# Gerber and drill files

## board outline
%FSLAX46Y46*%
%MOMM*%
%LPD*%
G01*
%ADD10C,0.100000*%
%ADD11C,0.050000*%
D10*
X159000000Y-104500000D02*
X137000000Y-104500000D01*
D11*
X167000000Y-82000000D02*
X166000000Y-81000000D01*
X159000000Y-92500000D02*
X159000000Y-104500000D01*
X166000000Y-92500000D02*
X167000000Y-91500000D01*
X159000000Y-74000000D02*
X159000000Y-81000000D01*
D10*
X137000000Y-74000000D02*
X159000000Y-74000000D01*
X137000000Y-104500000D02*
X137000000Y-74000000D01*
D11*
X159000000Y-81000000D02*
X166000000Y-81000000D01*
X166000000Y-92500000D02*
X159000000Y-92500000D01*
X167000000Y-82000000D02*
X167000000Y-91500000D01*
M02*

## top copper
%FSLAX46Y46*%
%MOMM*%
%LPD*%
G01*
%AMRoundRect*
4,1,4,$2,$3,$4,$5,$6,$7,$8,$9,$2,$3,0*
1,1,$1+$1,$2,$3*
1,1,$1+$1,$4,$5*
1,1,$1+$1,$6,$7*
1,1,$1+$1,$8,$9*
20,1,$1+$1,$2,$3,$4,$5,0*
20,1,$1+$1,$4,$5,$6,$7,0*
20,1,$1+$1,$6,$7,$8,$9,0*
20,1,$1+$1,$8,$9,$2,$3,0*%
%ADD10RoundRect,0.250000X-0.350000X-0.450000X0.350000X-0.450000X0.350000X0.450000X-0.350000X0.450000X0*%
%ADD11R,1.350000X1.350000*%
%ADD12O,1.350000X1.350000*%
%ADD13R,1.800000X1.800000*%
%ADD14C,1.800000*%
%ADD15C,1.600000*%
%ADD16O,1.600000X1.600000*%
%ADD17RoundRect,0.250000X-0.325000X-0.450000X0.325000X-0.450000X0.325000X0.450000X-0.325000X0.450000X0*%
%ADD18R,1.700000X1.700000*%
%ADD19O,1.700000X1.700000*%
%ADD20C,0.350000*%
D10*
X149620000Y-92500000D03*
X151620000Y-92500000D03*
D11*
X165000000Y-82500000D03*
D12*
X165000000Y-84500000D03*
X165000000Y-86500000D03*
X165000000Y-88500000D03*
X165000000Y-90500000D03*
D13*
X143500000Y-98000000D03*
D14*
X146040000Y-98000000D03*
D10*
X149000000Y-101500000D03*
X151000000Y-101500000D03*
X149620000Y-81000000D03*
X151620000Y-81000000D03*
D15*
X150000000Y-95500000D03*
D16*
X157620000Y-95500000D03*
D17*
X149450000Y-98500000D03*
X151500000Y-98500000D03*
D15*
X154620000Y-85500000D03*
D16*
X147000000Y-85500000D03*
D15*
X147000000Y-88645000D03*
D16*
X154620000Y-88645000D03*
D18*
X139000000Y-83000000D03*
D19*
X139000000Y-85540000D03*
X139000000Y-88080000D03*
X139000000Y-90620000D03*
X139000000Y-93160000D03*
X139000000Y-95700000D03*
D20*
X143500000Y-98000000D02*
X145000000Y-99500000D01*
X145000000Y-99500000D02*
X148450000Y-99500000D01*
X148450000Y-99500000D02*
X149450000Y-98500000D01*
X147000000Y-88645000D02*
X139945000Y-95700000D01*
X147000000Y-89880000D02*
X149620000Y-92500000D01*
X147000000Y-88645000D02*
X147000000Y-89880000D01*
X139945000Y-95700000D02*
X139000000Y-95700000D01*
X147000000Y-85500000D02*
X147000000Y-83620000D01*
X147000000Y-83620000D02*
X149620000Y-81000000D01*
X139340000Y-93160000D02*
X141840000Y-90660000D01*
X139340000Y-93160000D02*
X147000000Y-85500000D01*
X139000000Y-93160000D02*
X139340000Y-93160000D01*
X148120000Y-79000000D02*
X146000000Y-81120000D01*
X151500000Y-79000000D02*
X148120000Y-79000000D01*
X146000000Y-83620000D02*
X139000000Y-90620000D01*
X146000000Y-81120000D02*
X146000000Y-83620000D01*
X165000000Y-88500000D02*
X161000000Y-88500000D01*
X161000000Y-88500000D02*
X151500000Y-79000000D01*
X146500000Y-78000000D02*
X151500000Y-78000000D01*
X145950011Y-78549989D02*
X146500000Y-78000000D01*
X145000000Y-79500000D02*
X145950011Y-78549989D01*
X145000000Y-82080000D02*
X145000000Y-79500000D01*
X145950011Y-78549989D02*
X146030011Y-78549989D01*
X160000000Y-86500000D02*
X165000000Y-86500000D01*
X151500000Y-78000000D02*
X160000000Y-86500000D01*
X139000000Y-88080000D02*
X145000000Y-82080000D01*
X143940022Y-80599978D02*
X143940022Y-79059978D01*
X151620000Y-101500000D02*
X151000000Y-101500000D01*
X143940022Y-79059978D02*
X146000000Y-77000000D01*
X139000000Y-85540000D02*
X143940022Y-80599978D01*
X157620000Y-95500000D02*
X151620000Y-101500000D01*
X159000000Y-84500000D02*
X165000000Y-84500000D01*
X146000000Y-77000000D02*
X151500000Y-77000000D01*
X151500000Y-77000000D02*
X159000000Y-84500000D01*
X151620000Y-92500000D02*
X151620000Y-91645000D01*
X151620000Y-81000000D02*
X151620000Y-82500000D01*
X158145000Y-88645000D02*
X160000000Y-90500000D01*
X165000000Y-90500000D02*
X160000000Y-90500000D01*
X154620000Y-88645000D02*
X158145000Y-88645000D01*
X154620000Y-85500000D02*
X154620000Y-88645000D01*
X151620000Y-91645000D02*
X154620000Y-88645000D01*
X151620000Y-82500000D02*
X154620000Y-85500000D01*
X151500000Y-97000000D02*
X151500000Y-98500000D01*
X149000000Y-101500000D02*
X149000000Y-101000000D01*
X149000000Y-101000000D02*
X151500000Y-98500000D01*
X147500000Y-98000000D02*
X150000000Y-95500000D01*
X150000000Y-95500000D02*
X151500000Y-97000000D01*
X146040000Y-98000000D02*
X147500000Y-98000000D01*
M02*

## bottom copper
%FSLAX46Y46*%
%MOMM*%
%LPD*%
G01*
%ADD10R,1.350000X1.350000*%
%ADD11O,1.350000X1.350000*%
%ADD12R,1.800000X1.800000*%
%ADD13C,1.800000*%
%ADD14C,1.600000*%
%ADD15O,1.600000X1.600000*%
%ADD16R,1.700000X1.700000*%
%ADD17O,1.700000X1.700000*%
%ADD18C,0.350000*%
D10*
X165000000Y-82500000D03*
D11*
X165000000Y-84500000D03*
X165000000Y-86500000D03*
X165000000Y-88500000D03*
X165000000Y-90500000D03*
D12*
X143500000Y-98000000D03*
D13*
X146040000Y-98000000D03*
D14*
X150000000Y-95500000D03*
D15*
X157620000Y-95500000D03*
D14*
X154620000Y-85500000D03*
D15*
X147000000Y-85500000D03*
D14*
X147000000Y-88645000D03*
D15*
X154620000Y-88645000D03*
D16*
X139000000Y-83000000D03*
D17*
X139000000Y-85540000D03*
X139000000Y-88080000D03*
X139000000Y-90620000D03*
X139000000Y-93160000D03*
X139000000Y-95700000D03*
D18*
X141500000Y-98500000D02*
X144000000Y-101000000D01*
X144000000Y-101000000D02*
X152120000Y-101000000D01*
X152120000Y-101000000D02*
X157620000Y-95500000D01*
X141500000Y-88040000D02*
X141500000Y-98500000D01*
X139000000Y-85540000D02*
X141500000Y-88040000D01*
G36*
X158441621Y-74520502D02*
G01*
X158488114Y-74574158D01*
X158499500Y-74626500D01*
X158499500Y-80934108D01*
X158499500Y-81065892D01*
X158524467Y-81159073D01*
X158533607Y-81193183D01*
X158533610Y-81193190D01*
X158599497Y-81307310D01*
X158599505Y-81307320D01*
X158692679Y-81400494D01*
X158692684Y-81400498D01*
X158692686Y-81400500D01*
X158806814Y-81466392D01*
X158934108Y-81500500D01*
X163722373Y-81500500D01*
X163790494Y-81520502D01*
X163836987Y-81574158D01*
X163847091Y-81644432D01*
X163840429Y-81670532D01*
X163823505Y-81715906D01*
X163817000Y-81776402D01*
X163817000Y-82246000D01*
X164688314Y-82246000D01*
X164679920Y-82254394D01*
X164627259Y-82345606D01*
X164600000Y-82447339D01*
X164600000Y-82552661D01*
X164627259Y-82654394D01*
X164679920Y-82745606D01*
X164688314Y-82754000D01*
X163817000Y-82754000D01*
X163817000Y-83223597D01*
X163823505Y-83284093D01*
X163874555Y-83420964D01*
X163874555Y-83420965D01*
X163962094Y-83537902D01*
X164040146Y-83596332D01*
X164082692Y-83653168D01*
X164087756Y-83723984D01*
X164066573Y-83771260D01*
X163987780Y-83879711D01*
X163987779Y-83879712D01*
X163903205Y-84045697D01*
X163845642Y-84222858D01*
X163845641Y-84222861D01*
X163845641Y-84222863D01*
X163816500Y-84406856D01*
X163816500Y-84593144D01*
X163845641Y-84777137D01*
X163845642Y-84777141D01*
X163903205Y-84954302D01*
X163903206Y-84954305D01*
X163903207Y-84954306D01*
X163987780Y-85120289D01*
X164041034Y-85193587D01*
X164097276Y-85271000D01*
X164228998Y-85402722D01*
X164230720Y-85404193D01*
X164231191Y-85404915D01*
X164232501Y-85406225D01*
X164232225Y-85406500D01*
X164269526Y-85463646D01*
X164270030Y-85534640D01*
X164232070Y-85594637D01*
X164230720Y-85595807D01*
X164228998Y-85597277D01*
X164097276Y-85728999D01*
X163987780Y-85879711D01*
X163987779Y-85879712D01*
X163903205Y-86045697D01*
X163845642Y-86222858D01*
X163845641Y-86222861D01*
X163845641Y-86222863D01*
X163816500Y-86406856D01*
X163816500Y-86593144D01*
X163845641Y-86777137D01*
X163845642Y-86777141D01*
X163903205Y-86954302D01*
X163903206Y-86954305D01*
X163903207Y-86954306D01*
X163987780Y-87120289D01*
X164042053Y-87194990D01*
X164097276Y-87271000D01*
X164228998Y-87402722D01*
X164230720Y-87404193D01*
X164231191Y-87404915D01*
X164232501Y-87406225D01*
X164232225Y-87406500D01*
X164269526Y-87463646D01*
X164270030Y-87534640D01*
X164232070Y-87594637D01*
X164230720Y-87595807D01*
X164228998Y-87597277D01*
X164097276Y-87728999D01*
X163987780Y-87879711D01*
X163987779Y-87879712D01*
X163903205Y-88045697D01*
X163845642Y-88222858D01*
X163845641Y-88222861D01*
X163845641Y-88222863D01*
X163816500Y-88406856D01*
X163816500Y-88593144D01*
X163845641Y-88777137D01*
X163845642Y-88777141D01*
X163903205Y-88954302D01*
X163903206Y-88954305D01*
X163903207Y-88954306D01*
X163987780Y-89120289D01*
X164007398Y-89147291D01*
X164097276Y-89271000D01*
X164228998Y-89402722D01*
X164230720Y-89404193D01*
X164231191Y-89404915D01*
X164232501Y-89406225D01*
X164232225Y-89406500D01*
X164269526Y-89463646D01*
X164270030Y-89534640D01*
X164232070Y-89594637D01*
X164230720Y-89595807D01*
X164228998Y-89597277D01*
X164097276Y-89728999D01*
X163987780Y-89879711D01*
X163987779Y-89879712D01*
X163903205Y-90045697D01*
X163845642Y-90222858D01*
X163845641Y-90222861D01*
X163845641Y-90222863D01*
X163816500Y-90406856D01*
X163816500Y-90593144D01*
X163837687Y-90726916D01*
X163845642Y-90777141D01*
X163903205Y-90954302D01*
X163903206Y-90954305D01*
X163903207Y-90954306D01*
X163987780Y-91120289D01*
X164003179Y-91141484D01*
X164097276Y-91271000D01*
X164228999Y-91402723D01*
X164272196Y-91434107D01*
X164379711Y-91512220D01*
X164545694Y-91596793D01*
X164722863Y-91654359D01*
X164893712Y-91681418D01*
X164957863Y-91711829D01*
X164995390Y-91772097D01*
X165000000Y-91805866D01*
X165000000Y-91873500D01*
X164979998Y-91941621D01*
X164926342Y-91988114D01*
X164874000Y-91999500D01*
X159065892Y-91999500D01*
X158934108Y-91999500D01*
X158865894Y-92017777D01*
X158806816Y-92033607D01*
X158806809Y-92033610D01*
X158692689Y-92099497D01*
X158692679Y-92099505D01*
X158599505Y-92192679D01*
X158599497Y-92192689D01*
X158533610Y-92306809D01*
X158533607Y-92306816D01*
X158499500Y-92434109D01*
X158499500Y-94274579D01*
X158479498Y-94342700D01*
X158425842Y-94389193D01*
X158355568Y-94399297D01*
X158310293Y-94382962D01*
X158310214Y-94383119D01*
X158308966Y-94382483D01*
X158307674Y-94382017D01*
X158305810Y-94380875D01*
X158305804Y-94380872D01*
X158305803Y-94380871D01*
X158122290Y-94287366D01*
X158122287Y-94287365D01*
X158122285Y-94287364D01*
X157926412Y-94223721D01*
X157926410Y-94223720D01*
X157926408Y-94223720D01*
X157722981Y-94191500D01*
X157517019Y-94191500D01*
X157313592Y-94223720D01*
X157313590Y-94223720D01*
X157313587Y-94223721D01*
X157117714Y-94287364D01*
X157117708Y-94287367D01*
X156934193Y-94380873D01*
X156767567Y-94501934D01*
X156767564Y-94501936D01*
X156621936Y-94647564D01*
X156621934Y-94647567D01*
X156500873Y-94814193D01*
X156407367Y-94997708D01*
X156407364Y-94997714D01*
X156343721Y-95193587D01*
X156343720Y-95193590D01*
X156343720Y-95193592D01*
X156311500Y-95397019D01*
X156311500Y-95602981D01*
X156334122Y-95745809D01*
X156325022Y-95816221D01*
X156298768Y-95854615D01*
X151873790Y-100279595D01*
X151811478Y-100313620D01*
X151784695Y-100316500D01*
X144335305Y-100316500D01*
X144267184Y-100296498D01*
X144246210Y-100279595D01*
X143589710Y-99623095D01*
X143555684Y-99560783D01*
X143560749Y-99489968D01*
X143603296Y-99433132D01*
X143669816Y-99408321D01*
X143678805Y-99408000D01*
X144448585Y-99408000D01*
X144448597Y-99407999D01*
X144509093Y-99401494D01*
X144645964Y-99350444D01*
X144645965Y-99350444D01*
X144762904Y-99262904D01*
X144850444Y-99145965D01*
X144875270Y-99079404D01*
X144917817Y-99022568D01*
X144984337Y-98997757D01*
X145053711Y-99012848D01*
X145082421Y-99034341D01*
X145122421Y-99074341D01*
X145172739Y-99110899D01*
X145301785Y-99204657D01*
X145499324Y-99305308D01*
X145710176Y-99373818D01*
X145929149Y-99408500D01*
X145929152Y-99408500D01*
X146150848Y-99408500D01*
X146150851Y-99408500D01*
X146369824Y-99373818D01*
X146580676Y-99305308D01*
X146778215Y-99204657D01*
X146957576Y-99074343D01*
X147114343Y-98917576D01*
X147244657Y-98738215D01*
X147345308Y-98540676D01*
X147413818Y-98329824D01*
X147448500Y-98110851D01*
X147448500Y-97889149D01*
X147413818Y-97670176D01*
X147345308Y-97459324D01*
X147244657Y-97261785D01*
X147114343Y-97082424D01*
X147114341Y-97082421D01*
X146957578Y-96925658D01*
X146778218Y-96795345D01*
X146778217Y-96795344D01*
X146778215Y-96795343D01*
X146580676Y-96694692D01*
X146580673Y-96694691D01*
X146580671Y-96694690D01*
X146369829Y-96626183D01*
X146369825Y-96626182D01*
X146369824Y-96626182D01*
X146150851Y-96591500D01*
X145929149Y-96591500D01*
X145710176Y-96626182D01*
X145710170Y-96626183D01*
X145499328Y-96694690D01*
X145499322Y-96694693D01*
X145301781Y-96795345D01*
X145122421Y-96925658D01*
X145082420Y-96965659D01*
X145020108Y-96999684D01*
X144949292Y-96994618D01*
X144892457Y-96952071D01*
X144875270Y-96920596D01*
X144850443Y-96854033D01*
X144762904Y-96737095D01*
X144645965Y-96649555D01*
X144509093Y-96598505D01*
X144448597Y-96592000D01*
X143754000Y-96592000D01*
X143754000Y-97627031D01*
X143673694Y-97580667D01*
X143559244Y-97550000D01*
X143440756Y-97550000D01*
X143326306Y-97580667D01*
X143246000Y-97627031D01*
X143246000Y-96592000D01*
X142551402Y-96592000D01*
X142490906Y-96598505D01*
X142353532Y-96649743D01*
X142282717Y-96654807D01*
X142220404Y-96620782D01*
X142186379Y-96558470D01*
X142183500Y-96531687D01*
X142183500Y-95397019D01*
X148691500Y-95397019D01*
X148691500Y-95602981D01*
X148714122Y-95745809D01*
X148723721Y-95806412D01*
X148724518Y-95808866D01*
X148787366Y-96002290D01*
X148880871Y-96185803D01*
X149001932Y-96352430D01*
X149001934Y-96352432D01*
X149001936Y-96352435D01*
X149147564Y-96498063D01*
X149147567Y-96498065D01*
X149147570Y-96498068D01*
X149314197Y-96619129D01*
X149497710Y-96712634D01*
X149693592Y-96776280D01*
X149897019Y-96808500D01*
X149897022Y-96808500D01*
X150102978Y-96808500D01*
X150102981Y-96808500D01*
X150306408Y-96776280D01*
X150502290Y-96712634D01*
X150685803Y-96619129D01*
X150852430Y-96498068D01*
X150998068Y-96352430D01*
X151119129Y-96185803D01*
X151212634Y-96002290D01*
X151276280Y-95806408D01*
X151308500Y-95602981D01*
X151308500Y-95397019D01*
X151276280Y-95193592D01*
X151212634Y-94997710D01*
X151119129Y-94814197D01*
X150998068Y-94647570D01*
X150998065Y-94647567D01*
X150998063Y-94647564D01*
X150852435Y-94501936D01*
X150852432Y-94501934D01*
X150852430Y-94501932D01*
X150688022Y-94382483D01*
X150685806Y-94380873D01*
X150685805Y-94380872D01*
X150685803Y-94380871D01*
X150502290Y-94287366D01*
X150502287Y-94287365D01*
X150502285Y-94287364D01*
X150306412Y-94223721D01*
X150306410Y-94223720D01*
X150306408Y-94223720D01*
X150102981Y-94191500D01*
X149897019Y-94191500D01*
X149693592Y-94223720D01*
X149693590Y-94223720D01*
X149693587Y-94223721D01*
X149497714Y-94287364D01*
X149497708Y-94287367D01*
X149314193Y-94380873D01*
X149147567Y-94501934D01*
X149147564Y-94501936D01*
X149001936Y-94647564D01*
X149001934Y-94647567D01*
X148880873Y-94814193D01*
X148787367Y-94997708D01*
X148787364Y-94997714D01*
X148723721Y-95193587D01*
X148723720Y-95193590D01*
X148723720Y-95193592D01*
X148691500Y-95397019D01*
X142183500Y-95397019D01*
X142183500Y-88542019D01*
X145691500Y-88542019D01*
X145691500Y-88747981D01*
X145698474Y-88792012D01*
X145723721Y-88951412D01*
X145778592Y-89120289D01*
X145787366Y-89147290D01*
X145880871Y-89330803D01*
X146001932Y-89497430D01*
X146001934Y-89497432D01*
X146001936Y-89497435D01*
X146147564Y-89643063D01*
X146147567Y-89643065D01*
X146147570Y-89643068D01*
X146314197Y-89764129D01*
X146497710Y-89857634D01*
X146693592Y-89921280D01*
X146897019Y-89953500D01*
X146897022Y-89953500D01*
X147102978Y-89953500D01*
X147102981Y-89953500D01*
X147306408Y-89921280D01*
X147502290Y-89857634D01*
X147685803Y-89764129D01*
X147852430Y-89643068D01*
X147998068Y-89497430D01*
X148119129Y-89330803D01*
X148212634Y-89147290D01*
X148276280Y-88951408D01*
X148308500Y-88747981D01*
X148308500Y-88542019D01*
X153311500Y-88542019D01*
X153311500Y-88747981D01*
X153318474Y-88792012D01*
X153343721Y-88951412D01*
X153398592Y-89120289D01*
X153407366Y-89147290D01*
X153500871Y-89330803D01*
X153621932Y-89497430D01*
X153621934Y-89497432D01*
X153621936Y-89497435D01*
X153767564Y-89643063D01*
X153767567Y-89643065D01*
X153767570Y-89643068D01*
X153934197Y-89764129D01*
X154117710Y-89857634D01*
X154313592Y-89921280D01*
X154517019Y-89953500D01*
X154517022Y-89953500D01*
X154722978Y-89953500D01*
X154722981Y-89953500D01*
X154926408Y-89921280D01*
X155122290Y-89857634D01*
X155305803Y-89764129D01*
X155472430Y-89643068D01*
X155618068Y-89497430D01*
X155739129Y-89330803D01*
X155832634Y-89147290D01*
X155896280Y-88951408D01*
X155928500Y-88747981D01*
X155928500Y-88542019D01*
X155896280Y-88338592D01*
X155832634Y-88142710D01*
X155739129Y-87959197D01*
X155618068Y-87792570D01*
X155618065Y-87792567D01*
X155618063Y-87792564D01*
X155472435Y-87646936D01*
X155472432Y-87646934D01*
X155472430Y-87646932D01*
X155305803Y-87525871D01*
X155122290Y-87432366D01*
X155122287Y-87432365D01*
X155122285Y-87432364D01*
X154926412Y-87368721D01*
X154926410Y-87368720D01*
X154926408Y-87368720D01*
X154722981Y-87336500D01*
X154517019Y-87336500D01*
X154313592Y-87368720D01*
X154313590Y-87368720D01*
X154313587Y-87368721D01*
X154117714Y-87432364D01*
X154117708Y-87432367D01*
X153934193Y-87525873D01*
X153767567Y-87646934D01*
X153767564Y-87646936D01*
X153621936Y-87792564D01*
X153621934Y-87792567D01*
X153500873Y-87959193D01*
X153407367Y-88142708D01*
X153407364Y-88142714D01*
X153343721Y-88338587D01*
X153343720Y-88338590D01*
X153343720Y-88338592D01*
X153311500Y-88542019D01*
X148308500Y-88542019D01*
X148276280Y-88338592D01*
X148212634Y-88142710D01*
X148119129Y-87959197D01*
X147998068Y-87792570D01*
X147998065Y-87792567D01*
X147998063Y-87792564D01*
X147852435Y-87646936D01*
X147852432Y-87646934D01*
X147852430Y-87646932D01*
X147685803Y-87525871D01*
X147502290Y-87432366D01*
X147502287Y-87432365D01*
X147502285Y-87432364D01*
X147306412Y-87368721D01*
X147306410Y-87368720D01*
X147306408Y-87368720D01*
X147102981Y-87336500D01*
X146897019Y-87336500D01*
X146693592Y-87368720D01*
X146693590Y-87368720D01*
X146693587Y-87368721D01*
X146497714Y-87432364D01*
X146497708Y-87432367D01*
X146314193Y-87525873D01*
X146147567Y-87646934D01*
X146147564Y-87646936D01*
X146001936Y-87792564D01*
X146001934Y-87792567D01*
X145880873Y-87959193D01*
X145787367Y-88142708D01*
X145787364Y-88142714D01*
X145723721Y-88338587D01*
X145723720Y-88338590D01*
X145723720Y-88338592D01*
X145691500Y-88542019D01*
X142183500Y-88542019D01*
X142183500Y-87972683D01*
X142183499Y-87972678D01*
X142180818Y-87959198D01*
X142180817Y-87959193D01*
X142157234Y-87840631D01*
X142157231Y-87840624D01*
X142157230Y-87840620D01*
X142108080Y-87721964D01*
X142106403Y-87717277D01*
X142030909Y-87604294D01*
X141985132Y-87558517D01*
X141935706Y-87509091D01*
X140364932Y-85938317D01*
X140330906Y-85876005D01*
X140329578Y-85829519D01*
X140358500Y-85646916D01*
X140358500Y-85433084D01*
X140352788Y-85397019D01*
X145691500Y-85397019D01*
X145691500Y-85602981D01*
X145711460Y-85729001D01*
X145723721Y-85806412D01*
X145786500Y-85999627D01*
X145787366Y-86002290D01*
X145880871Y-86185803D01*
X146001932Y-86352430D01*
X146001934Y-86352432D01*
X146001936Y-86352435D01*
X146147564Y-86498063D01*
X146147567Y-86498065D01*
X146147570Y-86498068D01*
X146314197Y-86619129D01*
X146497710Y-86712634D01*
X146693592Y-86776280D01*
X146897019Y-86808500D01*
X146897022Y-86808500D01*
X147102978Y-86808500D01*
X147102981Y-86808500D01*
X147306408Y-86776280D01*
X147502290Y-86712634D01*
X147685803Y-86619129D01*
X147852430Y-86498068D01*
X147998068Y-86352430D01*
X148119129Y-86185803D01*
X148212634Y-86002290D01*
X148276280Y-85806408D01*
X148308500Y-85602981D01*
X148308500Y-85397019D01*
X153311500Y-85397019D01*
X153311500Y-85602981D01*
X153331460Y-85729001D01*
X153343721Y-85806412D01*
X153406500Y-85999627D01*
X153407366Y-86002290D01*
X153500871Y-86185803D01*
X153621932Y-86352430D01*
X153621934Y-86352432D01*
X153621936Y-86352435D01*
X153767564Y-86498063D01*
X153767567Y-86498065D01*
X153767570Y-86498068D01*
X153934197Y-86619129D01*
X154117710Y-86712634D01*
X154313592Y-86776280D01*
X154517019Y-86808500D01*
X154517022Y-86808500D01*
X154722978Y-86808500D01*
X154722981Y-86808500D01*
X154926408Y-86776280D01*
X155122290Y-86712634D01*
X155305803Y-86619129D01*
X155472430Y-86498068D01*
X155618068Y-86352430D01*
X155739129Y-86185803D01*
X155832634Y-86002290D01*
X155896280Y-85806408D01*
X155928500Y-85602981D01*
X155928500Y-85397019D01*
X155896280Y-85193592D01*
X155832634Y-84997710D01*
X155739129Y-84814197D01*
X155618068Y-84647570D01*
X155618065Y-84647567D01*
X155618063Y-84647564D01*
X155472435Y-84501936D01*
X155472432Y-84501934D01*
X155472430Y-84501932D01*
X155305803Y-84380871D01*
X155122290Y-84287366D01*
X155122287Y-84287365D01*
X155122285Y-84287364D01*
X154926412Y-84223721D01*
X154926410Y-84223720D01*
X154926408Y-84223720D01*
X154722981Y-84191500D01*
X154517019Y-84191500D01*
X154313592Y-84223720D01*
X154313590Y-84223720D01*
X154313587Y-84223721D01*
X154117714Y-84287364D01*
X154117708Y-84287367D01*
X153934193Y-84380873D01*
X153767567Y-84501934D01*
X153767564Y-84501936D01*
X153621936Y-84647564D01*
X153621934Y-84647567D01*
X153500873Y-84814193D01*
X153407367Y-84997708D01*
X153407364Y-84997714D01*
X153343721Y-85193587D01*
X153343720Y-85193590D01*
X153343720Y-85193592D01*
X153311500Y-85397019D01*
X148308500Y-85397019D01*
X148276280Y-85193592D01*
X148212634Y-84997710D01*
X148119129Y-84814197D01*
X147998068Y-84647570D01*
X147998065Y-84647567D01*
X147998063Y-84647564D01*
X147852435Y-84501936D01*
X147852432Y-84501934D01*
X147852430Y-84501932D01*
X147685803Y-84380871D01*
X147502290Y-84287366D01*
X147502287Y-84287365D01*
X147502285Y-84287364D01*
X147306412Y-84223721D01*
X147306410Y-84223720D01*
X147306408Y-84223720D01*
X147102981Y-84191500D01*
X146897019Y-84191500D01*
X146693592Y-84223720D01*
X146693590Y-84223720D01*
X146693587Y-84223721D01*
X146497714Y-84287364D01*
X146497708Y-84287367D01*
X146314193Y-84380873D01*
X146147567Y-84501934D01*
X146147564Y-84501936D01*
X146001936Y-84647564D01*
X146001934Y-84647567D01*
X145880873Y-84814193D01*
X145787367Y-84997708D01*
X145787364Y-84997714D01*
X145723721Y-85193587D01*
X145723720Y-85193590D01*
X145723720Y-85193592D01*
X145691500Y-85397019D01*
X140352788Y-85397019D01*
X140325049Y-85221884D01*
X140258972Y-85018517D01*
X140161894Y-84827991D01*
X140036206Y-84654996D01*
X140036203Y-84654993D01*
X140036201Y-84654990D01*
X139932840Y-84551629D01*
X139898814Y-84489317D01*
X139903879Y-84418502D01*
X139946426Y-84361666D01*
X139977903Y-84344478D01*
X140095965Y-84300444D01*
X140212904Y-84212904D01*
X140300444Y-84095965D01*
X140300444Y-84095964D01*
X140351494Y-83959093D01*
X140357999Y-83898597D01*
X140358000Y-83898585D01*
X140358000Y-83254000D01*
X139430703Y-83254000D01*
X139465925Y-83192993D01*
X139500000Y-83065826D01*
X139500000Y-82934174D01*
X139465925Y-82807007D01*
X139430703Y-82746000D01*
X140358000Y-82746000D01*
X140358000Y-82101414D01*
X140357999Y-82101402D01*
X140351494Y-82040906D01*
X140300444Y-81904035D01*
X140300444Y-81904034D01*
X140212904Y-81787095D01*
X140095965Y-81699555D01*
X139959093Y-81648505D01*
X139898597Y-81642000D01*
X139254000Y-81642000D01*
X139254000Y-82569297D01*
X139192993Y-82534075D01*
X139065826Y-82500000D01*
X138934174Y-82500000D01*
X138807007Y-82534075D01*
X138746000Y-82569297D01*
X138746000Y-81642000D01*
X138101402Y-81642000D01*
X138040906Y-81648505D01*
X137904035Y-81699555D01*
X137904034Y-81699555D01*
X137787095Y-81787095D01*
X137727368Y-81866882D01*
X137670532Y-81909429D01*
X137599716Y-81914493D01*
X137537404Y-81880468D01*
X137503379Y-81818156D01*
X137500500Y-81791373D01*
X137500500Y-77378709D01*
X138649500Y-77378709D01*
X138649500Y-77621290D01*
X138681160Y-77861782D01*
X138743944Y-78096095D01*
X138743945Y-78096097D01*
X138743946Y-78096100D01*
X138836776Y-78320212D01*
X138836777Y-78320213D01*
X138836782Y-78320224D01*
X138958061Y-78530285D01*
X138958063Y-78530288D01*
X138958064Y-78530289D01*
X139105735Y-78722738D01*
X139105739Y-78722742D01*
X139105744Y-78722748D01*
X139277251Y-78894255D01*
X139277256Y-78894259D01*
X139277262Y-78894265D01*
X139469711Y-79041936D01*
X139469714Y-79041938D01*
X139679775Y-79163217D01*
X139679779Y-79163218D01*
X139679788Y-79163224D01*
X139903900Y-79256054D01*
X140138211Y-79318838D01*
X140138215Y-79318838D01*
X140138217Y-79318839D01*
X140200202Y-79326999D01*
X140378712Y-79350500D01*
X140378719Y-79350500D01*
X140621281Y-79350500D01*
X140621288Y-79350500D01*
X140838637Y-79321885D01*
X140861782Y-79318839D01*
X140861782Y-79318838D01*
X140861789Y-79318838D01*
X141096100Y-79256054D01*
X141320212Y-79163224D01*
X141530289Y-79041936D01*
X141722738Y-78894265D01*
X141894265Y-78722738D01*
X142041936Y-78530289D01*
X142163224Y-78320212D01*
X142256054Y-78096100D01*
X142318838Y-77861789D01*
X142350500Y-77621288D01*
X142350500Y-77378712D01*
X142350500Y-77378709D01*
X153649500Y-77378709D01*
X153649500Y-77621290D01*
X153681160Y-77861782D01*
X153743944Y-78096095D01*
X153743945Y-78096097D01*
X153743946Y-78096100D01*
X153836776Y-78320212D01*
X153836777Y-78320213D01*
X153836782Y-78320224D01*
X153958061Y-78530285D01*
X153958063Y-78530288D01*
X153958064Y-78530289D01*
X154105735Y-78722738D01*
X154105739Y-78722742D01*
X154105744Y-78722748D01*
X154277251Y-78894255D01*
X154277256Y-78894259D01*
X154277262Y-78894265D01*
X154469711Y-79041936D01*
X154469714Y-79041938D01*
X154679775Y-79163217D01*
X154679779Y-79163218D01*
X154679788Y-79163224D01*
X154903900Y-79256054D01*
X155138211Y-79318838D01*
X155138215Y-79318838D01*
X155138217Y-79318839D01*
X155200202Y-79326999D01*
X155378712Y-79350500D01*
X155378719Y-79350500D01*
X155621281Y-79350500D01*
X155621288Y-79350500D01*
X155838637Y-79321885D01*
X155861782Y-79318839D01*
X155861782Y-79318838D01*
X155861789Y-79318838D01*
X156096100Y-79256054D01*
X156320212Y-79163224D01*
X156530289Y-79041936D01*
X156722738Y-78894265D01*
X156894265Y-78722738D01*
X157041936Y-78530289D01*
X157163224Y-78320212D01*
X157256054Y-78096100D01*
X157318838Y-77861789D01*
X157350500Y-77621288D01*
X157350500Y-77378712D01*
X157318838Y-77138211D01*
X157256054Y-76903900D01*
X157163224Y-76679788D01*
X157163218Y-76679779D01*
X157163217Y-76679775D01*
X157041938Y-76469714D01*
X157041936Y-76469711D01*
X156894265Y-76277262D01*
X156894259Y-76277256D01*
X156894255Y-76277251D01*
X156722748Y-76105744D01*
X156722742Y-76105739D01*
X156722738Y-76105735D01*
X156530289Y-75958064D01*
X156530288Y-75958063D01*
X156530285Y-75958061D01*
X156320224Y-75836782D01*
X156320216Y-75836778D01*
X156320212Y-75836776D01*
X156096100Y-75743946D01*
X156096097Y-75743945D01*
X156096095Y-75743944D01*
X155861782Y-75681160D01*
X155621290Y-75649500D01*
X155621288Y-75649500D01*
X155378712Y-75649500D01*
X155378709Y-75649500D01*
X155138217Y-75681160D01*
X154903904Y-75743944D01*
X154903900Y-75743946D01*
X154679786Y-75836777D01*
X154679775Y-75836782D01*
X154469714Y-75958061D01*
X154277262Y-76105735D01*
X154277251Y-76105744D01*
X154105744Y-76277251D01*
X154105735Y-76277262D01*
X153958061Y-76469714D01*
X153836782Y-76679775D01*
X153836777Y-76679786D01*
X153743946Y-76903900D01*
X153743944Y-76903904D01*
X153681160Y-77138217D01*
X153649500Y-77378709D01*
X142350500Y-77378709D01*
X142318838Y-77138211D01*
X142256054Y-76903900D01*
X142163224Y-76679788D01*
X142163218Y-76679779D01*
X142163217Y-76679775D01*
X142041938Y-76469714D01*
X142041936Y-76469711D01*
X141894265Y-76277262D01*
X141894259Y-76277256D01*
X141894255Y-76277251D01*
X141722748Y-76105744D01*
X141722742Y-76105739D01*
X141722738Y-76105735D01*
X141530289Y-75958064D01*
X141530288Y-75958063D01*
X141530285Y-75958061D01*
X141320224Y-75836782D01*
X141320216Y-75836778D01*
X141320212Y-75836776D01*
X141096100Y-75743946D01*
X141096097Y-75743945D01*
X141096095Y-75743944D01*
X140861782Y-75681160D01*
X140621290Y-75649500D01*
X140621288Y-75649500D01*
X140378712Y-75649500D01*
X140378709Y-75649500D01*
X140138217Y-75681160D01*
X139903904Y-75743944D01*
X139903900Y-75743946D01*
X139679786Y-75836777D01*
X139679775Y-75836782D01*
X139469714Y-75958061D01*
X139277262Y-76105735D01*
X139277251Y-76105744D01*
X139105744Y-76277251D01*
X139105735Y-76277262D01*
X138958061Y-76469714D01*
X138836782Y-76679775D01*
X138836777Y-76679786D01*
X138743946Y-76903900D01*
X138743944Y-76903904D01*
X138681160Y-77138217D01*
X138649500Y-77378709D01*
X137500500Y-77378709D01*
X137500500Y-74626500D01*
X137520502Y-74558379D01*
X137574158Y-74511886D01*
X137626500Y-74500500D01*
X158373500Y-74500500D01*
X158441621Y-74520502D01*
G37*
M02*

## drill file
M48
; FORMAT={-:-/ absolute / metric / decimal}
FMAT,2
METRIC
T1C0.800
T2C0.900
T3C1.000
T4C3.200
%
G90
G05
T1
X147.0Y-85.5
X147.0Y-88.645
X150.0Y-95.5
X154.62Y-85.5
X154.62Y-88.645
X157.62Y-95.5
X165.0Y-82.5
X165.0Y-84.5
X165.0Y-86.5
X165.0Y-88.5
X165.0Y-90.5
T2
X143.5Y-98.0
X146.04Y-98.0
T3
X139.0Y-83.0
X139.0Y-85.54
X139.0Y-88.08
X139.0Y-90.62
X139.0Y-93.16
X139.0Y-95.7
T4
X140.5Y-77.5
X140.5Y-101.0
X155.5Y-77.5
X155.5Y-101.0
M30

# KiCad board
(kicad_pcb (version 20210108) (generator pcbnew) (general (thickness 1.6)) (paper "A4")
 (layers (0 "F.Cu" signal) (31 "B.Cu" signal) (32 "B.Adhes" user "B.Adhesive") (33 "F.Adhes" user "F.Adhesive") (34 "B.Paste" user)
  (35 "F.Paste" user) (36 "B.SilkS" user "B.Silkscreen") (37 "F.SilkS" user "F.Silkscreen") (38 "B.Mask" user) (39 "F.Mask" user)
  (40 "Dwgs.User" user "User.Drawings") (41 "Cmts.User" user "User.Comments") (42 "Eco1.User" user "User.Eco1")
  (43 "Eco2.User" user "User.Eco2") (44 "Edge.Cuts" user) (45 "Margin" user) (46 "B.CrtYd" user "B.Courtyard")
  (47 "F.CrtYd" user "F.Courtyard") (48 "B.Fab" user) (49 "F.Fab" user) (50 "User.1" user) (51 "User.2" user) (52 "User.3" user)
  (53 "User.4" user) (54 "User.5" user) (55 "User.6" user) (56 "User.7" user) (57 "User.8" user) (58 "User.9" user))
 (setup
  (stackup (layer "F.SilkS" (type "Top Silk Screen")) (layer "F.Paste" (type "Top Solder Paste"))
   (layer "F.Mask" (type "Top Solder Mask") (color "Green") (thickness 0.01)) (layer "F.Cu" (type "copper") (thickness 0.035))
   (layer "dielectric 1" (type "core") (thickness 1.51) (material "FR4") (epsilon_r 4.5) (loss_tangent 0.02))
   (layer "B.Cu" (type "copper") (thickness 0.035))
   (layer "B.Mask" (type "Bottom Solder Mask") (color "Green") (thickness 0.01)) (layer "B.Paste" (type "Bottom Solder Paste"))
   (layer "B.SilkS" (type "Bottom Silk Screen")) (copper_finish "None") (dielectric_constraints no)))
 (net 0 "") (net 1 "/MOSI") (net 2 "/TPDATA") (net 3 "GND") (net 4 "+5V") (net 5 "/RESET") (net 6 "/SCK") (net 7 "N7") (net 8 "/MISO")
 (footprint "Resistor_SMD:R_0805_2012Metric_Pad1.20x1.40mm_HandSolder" (layer "F.Cu") (at 150.62 92.5)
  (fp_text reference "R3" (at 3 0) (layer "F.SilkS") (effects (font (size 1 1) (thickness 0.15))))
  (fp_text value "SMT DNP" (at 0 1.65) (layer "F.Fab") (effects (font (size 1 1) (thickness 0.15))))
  (pad "1" smd roundrect (at -1 0) (locked) (size 1.2 1.4) (layers "F.Cu" "F.Paste" "F.Mask") (roundrect_rratio 0.2083333333333333)
   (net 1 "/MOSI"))
  (pad "2" smd roundrect (at 1 0) (locked) (size 1.2 1.4) (layers "F.Cu" "F.Paste" "F.Mask") (roundrect_rratio 0.2083333333333333)
   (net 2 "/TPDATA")))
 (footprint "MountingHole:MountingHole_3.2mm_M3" (layer "F.Cu") (at 140.5 101)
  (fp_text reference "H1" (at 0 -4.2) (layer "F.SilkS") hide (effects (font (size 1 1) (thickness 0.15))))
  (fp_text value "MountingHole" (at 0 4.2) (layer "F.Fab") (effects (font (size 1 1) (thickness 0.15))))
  (pad "1" np_thru_hole circle (at 0 0) (locked) (size 3.2 3.2) (drill 3.2) (layers *.Cu *.Mask)))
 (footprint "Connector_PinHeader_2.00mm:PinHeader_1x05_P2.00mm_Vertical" (layer "F.Cu") (at 165 82.5)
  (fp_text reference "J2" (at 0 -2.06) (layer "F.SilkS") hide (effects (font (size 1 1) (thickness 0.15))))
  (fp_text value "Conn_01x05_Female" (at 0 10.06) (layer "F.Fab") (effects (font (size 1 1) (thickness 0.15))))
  (pad "1" thru_hole rect (at 0 0) (locked) (size 1.35 1.35) (drill 0.8) (layers *.Cu *.Mask) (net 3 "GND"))
  (pad "2" thru_hole oval (at 0 2) (locked) (size 1.35 1.35) (drill 0.8) (layers *.Cu *.Mask) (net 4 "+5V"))
  (pad "3" thru_hole oval (at 0 4) (locked) (size 1.35 1.35) (drill 0.8) (layers *.Cu *.Mask) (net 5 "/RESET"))
  (pad "4" thru_hole oval (at 0 6) (locked) (size 1.35 1.35) (drill 0.8) (layers *.Cu *.Mask) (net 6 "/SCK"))
  (pad "5" thru_hole oval (at 0 8) (locked) (size 1.35 1.35) (drill 0.8) (layers *.Cu *.Mask) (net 2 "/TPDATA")))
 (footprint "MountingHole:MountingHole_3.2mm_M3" (layer "F.Cu") (at 140.5 77.5)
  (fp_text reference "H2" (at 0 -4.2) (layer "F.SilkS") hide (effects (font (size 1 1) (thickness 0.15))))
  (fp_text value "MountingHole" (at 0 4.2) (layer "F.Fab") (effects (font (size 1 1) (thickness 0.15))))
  (pad "1" np_thru_hole circle (at 0 0) (locked) (size 3.2 3.2) (drill 3.2) (layers *.Cu *.Mask)))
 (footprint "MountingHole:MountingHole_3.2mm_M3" (layer "F.Cu") (at 155.5 101)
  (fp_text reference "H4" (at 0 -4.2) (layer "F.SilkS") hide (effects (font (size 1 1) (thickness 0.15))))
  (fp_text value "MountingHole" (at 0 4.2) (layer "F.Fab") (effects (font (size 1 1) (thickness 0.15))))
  (pad "1" np_thru_hole circle (at 0 0) (locked) (size 3.2 3.2) (drill 3.2) (layers *.Cu *.Mask)))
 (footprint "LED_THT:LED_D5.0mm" (layer "F.Cu") (at 143.5 98)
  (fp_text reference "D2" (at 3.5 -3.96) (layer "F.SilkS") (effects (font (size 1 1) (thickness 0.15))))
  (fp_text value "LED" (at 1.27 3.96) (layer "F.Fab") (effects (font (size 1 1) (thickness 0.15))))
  (pad "1" thru_hole rect (at 0 0) (locked) (size 1.8 1.8) (drill 0.9) (layers *.Cu *.Mask) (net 3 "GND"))
  (pad "2" thru_hole circle (at 2.54 0) (locked) (size 1.8 1.8) (drill 0.9) (layers *.Cu *.Mask) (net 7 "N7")))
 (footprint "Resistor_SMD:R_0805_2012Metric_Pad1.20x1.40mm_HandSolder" (layer "F.Cu") (at 150 101.5)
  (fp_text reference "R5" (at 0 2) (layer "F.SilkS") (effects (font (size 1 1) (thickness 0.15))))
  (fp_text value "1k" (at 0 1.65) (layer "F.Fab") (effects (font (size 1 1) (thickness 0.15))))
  (pad "1" smd roundrect (at -1 0) (locked) (size 1.2 1.4) (layers "F.Cu" "F.Paste" "F.Mask") (roundrect_rratio 0.2083333333333333)
   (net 7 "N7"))
  (pad "2" smd roundrect (at 1 0) (locked) (size 1.2 1.4) (layers "F.Cu" "F.Paste" "F.Mask") (roundrect_rratio 0.2083333333333333)
   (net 4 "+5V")))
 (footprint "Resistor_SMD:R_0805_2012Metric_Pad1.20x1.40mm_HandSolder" (layer "F.Cu") (at 150.62 81)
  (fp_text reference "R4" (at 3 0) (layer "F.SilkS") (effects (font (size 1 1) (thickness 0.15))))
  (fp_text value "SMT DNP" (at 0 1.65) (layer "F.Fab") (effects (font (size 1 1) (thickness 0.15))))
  (pad "1" smd roundrect (at -1 0) (locked) (size 1.2 1.4) (layers "F.Cu" "F.Paste" "F.Mask") (roundrect_rratio 0.2083333333333333)
   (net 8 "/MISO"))
  (pad "2" smd roundrect (at 1 0) (locked) (size 1.2 1.4) (layers "F.Cu" "F.Paste" "F.Mask") (roundrect_rratio 0.2083333333333333)
   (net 2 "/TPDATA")))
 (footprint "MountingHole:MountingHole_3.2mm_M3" (layer "F.Cu") (at 155.5 77.5)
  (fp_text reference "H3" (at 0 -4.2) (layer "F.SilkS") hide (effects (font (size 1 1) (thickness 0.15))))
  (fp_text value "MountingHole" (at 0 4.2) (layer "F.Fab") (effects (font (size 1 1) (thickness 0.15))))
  (pad "1" np_thru_hole circle (at 0 0) (locked) (size 3.2 3.2) (drill 3.2) (layers *.Cu *.Mask)))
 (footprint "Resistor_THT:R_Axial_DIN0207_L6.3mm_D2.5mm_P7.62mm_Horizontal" (layer "F.Cu") (at 150 95.5)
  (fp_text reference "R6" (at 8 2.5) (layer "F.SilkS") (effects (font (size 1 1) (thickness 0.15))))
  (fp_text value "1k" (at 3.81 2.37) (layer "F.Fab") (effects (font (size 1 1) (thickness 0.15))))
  (pad "1" thru_hole circle (at 0 0) (locked) (size 1.6 1.6) (drill 0.8) (layers *.Cu *.Mask) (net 7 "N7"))
  (pad "2" thru_hole oval (at 7.62 0) (locked) (size 1.6 1.6) (drill 0.8) (layers *.Cu *.Mask) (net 4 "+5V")))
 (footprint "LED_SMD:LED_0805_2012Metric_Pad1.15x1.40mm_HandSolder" (layer "F.Cu") (at 150.475 98.5)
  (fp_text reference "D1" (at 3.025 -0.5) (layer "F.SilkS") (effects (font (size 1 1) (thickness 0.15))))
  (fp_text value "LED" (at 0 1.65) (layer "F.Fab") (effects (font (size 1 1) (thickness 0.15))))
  (pad "1" smd roundrect (at -1.025 0) (locked) (size 1.15 1.4) (layers "F.Cu" "F.Paste" "F.Mask") (roundrect_rratio 0.2173913043478261)
   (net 3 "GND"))
  (pad "2" smd roundrect (at 1.025 0) (locked) (size 1.15 1.4) (layers "F.Cu" "F.Paste" "F.Mask") (roundrect_rratio 0.2173913043478261)
   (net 7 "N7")))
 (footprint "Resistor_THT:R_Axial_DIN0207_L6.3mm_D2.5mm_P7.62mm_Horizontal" (layer "F.Cu") (at 154.62 85.5 180)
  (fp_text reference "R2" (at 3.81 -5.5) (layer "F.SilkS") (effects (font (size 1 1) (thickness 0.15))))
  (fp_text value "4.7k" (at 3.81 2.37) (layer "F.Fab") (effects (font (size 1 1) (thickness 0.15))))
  (pad "1" thru_hole circle (at 0 0 180) (locked) (size 1.6 1.6) (drill 0.8) (layers *.Cu *.Mask) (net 2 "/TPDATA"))
  (pad "2" thru_hole oval (at 7.62 0 180) (locked) (size 1.6 1.6) (drill 0.8) (layers *.Cu *.Mask) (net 8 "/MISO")))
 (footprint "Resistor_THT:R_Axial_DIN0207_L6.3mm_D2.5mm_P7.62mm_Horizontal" (layer "F.Cu") (at 147 88.645)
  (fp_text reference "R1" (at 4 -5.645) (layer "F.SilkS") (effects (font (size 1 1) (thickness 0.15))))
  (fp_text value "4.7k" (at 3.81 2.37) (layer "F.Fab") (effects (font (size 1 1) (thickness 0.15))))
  (pad "1" thru_hole circle (at 0 0) (locked) (size 1.6 1.6) (drill 0.8) (layers *.Cu *.Mask) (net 1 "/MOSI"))
  (pad "2" thru_hole oval (at 7.62 0) (locked) (size 1.6 1.6) (drill 0.8) (layers *.Cu *.Mask) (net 2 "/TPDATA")))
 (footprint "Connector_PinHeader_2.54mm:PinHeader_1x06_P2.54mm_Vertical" (layer "B.Cu") (at 139 83 180)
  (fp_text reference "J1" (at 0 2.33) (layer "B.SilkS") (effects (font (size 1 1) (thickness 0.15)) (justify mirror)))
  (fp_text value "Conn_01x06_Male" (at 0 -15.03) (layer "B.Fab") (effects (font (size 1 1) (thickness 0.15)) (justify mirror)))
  (pad "1" thru_hole rect (at 0 0 180) (locked) (size 1.7 1.7) (drill 1) (layers *.Cu *.Mask) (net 3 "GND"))
  (pad "2" thru_hole oval (at 0 -2.54 180) (locked) (size 1.7 1.7) (drill 1) (layers *.Cu *.Mask) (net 4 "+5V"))
  (pad "3" thru_hole oval (at 0 -5.08 180) (locked) (size 1.7 1.7) (drill 1) (layers *.Cu *.Mask) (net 5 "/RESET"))
  (pad "4" thru_hole oval (at 0 -7.62 180) (locked) (size 1.7 1.7) (drill 1) (layers *.Cu *.Mask) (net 6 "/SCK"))
  (pad "5" thru_hole oval (at 0 -10.16 180) (locked) (size 1.7 1.7) (drill 1) (layers *.Cu *.Mask) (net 8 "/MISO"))
  (pad "6" thru_hole oval (at 0 -12.7 180) (locked) (size 1.7 1.7) (drill 1) (layers *.Cu *.Mask) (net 1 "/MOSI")))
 (gr_line (start 159 104.5) (end 137 104.5) (layer "Edge.Cuts") (width 0.1))
 (gr_line (start 167 82) (end 166 81) (layer "Edge.Cuts") (width 0.05))
 (gr_line (start 159 92.5) (end 159 104.5) (layer "Edge.Cuts") (width 0.05))
 (gr_line (start 166 92.5) (end 167 91.5) (layer "Edge.Cuts") (width 0.05))
 (gr_line (start 159 74) (end 159 81) (layer "Edge.Cuts") (width 0.05))
 (gr_line (start 137 74) (end 159 74) (layer "Edge.Cuts") (width 0.1))
 (gr_line (start 137 104.5) (end 137 74) (layer "Edge.Cuts") (width 0.1))
 (gr_line (start 159 81) (end 166 81) (layer "Edge.Cuts") (width 0.05))
 (gr_line (start 166 92.5) (end 159 92.5) (layer "Edge.Cuts") (width 0.05))
 (gr_line (start 167 82) (end 167 91.5) (layer "Edge.Cuts") (width 0.05))
 (segment (start 143.5 98) (end 145 99.5) (width 0.35) (layer "F.Cu") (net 3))
 (segment (start 145 99.5) (end 148.45 99.5) (width 0.35) (layer "F.Cu") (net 3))
 (segment (start 148.45 99.5) (end 149.45 98.5) (width 0.35) (layer "F.Cu") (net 3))
 (segment (start 147 88.645) (end 139.945 95.7) (width 0.35) (layer "F.Cu") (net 1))
 (segment (start 147 89.88) (end 149.62 92.5) (width 0.35) (layer "F.Cu") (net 1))
 (segment (start 147 88.645) (end 147 89.88) (width 0.35) (layer "F.Cu") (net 1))
 (segment (start 139.945 95.7) (end 139 95.7) (width 0.35) (layer "F.Cu") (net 1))
 (segment (start 147 85.5) (end 147 83.62) (width 0.35) (layer "F.Cu") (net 8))
 (segment (start 147 83.62) (end 149.62 81) (width 0.35) (layer "F.Cu") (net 8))
 (segment (start 139.34 93.16) (end 141.84 90.66) (width 0.35) (layer "F.Cu") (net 8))
 (segment (start 139.34 93.16) (end 147 85.5) (width 0.35) (layer "F.Cu") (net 8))
 (segment (start 139 93.16) (end 139.34 93.16) (width 0.35) (layer "F.Cu") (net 8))
 (segment (start 148.12 79) (end 146 81.12) (width 0.35) (layer "F.Cu") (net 6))
 (segment (start 151.5 79) (end 148.12 79) (width 0.35) (layer "F.Cu") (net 6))
 (segment (start 146 83.62) (end 139 90.62) (width 0.35) (layer "F.Cu") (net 6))
 (segment (start 146 81.12) (end 146 83.62) (width 0.35) (layer "F.Cu") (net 6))
 (segment (start 165 88.5) (end 161 88.5) (width 0.35) (layer "F.Cu") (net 6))
 (segment (start 161 88.5) (end 151.5 79) (width 0.35) (layer "F.Cu") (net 6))
 (segment (start 146.5 78) (end 151.5 78) (width 0.35) (layer "F.Cu") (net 5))
 (segment (start 145.950011 78.549989) (end 146.5 78) (width 0.35) (layer "F.Cu") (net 5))
 (segment (start 145 79.5) (end 145.950011 78.549989) (width 0.35) (layer "F.Cu") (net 5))
 (segment (start 145 82.08) (end 145 79.5) (width 0.35) (layer "F.Cu") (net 5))
 (segment (start 145.950011 78.549989) (end 146.030011 78.549989) (width 0.35) (layer "F.Cu") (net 5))
 (segment (start 160 86.5) (end 165 86.5) (width 0.35) (layer "F.Cu") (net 5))
 (segment (start 151.5 78) (end 160 86.5) (width 0.35) (layer "F.Cu") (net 5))
 (segment (start 139 88.08) (end 145 82.08) (width 0.35) (layer "F.Cu") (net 5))
 (segment (start 143.940022 80.599978) (end 143.940022 79.059978) (width 0.35) (layer "F.Cu") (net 4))
 (segment (start 151.62 101.5) (end 151 101.5) (width 0.35) (layer "F.Cu") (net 4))
 (segment (start 143.940022 79.059978) (end 146 77) (width 0.35) (layer "F.Cu") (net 4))
 (segment (start 139 85.54) (end 143.940022 80.599978) (width 0.35) (layer "F.Cu") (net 4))
 (segment (start 157.62 95.5) (end 151.62 101.5) (width 0.35) (layer "F.Cu") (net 4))
 (segment (start 159 84.5) (end 165 84.5) (width 0.35) (layer "F.Cu") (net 4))
 (segment (start 146 77) (end 151.5 77) (width 0.35) (layer "F.Cu") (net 4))
 (segment (start 151.5 77) (end 159 84.5) (width 0.35) (layer "F.Cu") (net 4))
 (segment (start 141.5 98.5) (end 144 101) (width 0.35) (layer "B.Cu") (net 4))
 (segment (start 144 101) (end 152.12 101) (width 0.35) (layer "B.Cu") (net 4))
 (segment (start 152.12 101) (end 157.62 95.5) (width 0.35) (layer "B.Cu") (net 4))
 (segment (start 141.5 88.04) (end 141.5 98.5) (width 0.35) (layer "B.Cu") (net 4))
 (segment (start 139 85.54) (end 141.5 88.04) (width 0.35) (layer "B.Cu") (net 4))
 (segment (start 151.62 92.5) (end 151.62 91.645) (width 0.35) (layer "F.Cu") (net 2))
 (segment (start 151.62 81) (end 151.62 82.5) (width 0.35) (layer "F.Cu") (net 2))
 (segment (start 158.145 88.645) (end 160 90.5) (width 0.35) (layer "F.Cu") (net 2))
 (segment (start 165 90.5) (end 160 90.5) (width 0.35) (layer "F.Cu") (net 2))
 (segment (start 154.62 88.645) (end 158.145 88.645) (width 0.35) (layer "F.Cu") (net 2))
 (segment (start 154.62 85.5) (end 154.62 88.645) (width 0.35) (layer "F.Cu") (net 2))
 (segment (start 151.62 91.645) (end 154.62 88.645) (width 0.35) (layer "F.Cu") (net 2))
 (segment (start 151.62 82.5) (end 154.62 85.5) (width 0.35) (layer "F.Cu") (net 2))
 (segment (start 151.5 97) (end 151.5 98.5) (width 0.35) (layer "F.Cu") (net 7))
 (segment (start 149 101.5) (end 149 101) (width 0.35) (layer "F.Cu") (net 7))
 (segment (start 149 101) (end 151.5 98.5) (width 0.35) (layer "F.Cu") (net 7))
 (segment (start 147.5 98) (end 150 95.5) (width 0.35) (layer "F.Cu") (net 7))
 (segment (start 150 95.5) (end 151.5 97) (width 0.35) (layer "F.Cu") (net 7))
 (segment (start 146.04 98) (end 147.5 98) (width 0.35) (layer "F.Cu") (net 7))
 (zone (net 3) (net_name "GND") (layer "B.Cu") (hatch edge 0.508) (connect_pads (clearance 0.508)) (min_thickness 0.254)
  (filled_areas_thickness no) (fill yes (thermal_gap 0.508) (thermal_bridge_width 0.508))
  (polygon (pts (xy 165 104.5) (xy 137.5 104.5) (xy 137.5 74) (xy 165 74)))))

